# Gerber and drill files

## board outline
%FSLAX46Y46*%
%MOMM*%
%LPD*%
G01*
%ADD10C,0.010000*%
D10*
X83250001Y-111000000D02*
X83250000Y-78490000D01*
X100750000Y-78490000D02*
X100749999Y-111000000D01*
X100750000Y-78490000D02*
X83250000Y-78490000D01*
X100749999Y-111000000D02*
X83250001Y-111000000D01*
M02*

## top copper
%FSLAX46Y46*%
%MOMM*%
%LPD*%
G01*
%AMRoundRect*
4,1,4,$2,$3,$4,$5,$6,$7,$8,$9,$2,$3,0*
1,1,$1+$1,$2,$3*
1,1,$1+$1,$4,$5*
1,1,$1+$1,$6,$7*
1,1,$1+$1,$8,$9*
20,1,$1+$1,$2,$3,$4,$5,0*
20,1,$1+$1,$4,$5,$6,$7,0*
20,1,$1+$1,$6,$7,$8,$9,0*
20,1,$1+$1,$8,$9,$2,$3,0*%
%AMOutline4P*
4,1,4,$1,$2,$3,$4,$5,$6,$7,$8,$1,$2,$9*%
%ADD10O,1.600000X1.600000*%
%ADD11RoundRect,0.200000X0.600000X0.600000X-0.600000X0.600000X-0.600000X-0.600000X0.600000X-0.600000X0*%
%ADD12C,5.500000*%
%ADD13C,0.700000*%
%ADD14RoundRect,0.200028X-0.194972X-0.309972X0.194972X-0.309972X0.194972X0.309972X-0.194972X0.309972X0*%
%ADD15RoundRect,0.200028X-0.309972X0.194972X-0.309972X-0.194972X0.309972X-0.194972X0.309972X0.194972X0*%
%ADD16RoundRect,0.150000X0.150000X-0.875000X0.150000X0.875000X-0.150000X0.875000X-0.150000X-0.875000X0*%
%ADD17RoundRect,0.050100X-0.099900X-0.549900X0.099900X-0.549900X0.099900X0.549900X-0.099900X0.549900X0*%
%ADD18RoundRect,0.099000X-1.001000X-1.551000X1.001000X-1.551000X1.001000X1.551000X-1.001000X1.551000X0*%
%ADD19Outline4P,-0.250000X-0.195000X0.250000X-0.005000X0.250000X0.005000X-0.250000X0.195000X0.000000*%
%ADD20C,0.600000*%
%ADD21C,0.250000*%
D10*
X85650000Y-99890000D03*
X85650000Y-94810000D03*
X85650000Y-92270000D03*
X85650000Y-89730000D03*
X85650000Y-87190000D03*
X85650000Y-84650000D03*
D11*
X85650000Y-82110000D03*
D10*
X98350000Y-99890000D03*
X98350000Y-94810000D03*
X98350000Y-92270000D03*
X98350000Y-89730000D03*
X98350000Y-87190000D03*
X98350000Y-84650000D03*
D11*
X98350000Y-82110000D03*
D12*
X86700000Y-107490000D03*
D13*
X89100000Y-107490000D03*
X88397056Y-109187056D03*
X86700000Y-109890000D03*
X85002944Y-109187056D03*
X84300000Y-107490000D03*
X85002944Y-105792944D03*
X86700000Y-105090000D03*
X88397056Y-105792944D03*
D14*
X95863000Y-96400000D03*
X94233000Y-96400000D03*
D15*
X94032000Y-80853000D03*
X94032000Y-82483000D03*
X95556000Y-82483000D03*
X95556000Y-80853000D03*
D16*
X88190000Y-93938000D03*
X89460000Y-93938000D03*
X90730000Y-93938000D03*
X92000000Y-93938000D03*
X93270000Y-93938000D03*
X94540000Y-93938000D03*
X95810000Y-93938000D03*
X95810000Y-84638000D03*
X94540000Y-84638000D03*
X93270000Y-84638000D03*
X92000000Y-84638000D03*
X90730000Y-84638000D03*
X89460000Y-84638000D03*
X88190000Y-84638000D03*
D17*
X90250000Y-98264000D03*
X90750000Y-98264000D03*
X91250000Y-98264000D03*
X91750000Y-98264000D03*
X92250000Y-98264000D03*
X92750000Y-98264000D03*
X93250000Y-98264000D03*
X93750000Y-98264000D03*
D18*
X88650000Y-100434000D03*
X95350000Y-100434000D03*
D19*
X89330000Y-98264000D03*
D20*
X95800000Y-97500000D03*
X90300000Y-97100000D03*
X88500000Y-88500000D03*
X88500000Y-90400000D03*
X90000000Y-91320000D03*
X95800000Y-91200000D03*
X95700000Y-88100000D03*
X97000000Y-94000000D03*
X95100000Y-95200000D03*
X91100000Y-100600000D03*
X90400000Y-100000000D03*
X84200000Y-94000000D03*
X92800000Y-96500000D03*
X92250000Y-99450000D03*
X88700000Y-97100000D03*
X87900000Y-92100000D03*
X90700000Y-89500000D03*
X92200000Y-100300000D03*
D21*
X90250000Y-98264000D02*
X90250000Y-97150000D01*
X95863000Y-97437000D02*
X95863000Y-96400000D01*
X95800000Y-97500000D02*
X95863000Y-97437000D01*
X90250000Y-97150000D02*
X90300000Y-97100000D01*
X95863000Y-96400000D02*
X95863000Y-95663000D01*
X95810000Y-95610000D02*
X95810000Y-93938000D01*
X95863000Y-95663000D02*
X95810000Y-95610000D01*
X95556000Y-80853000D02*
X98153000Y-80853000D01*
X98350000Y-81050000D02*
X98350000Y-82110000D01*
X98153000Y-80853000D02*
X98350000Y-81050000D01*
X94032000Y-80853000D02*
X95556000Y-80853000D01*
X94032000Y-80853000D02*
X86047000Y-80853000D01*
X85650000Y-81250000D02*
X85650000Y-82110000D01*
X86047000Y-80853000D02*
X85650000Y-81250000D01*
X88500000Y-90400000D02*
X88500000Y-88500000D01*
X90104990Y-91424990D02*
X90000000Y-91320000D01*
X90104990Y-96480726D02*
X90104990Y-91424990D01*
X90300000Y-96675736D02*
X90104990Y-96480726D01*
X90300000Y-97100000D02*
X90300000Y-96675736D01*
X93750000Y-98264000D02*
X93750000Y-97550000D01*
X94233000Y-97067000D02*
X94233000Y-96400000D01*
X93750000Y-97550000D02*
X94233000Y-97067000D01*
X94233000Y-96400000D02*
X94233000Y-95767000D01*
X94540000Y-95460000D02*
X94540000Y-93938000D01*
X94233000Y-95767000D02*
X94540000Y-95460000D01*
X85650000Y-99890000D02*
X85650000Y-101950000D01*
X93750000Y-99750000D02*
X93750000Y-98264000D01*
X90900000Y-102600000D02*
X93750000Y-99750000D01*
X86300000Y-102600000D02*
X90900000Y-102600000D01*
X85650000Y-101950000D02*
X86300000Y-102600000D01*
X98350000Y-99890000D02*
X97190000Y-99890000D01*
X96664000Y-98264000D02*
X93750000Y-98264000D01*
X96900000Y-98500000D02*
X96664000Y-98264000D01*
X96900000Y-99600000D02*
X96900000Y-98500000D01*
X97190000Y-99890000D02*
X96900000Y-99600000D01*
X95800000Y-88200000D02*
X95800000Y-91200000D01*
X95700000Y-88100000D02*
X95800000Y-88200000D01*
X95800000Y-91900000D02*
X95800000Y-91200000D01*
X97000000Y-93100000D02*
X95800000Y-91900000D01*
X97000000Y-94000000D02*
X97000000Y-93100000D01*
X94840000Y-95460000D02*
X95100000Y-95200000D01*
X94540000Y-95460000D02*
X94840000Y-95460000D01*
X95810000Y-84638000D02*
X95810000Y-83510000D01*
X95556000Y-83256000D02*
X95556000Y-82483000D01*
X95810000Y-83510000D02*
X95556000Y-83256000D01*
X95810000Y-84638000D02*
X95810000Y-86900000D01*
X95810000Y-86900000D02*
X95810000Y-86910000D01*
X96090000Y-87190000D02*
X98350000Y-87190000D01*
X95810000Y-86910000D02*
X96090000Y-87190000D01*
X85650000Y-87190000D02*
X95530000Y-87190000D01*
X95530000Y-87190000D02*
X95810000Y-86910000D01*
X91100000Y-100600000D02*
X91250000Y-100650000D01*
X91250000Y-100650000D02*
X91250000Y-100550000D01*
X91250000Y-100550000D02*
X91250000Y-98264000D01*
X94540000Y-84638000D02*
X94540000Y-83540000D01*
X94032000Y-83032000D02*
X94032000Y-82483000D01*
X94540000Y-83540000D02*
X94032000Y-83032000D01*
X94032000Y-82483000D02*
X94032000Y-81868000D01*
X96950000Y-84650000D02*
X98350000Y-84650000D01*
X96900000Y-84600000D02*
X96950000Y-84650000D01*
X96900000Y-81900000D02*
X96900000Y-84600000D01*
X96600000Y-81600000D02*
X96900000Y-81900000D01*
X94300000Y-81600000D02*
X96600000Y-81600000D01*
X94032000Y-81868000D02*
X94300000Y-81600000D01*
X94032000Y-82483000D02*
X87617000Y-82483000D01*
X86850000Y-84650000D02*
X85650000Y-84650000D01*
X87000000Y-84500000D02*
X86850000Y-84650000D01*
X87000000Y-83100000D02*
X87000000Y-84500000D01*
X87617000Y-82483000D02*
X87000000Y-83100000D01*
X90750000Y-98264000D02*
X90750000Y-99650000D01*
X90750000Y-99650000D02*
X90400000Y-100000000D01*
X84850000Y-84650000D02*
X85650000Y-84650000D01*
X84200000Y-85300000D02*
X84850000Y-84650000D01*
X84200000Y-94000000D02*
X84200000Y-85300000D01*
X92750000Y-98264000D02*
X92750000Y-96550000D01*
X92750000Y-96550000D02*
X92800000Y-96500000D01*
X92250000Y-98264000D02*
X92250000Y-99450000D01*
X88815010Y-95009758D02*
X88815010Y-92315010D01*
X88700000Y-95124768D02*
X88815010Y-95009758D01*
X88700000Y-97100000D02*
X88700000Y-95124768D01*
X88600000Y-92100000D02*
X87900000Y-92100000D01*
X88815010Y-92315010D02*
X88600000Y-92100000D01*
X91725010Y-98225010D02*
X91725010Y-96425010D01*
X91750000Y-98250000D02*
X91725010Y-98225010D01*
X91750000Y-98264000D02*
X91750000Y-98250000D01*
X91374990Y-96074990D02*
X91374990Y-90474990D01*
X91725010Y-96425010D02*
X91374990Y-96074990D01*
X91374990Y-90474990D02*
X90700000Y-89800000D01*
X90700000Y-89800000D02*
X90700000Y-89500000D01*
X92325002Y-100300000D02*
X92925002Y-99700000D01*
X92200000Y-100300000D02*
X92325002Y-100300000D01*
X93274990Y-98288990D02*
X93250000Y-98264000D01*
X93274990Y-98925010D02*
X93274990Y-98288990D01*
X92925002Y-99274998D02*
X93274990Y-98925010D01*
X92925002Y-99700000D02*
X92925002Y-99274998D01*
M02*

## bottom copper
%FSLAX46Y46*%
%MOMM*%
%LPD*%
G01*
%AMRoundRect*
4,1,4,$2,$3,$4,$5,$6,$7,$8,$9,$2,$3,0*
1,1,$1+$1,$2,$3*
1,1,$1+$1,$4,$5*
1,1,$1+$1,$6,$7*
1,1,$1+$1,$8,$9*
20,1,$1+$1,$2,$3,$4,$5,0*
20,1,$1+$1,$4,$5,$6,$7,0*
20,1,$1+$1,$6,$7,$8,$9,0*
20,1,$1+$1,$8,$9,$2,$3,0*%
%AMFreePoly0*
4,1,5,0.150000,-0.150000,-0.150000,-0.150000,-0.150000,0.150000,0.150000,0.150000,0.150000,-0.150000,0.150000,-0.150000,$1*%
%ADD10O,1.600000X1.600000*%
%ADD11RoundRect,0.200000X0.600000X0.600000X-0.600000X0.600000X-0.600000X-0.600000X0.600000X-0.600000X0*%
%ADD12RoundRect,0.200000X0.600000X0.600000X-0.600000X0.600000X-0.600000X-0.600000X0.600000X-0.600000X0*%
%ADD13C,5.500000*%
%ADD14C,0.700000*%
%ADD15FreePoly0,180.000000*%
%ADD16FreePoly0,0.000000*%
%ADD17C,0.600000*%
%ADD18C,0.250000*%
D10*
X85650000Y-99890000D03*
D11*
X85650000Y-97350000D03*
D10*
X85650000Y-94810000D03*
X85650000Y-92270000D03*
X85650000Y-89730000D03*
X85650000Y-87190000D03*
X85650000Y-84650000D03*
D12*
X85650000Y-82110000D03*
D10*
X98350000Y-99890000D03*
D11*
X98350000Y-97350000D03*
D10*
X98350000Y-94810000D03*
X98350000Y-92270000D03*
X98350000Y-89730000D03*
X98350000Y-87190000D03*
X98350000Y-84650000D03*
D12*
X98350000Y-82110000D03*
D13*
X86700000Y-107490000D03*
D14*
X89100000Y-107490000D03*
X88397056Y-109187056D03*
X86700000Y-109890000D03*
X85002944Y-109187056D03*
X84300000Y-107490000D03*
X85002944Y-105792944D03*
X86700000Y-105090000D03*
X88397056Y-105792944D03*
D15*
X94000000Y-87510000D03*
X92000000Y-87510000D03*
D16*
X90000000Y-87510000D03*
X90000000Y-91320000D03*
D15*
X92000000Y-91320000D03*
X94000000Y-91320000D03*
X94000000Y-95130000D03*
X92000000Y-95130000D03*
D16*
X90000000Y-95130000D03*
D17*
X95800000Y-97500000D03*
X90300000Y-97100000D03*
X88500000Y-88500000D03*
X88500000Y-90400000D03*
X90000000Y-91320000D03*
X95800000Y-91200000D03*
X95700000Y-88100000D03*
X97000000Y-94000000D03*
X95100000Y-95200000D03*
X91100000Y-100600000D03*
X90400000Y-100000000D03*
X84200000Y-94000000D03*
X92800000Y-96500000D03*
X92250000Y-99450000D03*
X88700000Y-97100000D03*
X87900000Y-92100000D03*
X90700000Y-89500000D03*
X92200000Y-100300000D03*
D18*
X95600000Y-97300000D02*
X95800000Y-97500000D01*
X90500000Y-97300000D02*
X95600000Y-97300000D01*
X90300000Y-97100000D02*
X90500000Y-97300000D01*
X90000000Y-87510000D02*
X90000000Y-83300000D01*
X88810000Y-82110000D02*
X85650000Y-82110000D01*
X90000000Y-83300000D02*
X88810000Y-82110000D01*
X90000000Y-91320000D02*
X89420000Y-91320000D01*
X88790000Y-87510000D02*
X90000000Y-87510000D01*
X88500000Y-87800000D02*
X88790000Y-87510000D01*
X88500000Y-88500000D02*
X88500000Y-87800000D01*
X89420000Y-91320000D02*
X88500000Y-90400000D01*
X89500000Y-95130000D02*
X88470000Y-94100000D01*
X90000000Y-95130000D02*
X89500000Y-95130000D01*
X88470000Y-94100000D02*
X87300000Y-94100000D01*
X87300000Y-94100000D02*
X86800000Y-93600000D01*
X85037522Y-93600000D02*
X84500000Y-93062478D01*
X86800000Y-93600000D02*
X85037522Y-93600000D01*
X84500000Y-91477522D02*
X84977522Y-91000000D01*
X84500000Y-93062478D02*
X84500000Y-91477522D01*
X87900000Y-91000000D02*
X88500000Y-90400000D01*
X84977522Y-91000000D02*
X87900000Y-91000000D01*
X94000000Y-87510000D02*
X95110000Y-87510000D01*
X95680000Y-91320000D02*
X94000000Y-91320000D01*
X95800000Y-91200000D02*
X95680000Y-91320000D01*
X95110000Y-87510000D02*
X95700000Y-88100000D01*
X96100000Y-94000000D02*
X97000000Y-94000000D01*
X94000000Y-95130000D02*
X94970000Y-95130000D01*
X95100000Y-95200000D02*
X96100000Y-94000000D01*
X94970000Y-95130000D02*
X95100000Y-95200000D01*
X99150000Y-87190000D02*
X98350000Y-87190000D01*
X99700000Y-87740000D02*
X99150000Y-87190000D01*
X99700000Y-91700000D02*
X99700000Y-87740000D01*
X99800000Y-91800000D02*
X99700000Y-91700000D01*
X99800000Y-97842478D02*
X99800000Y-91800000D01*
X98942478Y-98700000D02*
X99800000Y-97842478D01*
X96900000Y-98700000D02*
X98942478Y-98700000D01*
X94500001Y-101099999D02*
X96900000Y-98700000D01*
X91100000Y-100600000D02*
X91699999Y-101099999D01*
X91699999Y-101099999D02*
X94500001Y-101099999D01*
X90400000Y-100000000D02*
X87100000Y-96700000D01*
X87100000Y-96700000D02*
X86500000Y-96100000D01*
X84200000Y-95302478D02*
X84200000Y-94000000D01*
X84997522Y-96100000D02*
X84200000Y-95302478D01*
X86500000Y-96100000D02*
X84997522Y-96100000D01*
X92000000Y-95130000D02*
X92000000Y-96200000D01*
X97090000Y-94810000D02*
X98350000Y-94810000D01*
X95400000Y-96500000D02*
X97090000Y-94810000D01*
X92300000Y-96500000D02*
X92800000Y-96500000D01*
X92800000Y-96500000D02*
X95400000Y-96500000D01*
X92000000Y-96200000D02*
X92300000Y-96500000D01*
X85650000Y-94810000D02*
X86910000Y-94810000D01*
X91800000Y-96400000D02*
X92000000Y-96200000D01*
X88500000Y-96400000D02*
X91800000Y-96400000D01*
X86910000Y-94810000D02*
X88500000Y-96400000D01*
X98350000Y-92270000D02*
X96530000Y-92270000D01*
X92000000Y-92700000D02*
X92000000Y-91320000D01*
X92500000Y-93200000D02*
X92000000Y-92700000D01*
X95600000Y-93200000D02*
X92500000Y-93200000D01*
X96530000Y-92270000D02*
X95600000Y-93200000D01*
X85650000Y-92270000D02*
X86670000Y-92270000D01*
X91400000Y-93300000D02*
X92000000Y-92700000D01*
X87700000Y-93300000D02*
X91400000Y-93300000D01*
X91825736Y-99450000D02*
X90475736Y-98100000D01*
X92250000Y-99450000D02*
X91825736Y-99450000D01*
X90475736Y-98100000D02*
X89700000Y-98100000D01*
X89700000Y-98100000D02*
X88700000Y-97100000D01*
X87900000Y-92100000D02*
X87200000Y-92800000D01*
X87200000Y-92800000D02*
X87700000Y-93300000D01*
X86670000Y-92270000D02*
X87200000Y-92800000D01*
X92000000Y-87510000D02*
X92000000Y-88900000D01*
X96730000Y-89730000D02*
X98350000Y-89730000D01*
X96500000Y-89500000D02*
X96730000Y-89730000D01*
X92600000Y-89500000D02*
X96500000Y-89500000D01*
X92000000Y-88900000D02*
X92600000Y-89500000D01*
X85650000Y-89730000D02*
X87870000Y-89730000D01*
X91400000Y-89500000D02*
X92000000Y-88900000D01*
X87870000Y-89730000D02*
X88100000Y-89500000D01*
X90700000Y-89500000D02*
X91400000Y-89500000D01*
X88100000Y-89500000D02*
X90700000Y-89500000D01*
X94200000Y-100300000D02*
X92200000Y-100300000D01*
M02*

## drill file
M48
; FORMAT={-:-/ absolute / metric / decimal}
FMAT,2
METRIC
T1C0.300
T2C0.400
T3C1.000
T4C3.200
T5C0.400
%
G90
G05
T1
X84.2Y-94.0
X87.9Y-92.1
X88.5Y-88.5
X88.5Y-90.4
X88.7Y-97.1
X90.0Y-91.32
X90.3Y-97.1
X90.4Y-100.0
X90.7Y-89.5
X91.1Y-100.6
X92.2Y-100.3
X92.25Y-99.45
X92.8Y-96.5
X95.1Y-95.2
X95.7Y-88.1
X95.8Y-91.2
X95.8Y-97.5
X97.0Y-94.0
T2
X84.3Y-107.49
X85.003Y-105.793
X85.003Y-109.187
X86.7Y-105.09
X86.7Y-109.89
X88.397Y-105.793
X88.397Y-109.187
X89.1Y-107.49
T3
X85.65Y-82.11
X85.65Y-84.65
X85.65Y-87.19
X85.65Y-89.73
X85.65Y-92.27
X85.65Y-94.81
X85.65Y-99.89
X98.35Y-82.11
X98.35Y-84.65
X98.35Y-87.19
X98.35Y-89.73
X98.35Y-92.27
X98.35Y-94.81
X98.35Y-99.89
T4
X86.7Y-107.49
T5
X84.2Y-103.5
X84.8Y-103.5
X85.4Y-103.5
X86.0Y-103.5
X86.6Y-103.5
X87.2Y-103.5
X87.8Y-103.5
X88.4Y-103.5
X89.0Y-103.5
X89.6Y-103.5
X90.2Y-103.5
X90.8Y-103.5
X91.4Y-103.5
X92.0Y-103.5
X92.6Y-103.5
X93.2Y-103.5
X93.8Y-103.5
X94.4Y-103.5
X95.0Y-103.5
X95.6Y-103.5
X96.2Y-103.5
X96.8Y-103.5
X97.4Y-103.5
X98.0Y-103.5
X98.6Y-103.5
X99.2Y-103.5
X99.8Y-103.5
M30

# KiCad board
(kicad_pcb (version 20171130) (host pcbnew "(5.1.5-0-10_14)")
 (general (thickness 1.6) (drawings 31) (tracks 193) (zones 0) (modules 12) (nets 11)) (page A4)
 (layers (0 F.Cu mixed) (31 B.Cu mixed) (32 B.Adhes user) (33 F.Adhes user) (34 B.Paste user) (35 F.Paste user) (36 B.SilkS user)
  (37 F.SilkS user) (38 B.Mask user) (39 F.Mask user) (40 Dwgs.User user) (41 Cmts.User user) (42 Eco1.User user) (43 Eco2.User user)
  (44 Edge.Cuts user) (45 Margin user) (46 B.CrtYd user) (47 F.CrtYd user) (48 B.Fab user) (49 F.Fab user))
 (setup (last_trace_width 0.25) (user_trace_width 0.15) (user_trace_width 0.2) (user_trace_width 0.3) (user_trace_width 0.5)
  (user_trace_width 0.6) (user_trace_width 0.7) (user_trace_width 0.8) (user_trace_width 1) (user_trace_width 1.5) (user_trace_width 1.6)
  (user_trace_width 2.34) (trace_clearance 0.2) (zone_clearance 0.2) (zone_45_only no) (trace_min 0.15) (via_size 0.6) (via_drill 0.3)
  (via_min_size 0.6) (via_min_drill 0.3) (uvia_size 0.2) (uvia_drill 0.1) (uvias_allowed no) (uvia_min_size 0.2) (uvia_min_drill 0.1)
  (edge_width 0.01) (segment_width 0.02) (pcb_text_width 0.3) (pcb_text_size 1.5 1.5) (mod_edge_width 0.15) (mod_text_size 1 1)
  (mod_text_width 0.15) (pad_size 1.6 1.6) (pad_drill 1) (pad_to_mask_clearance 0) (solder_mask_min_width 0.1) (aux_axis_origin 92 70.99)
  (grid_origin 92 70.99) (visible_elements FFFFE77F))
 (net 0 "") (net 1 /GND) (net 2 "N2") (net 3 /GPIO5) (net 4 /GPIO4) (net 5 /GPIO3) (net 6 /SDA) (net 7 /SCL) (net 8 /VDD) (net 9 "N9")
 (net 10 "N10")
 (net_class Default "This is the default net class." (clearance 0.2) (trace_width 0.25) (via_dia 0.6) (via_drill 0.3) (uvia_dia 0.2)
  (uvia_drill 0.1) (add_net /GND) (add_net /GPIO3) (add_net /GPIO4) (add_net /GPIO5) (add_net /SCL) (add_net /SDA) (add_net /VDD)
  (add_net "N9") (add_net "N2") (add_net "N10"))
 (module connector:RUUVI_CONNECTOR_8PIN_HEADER (layer B.Cu) (at 85.65 82.11 180)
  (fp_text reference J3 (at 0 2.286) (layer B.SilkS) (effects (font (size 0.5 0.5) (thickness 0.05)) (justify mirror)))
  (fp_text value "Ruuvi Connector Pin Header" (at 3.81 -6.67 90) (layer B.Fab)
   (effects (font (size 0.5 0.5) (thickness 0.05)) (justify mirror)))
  (pad 8 thru_hole oval (at 0 -17.78 180) (size 1.6 1.6) (drill 1) (layers *.Cu *.Mask) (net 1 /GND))
  (pad 7 smd roundrect (at 0 -15.24 180) (size 1.6 1.6) (layers B.Cu B.Paste B.Mask) (roundrect_rratio 0.125) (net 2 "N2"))
  (pad 6 thru_hole oval (at 0 -12.7 180) (size 1.6 1.6) (drill 1) (layers *.Cu *.Mask) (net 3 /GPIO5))
  (pad 5 thru_hole oval (at 0 -10.16 180) (size 1.6 1.6) (drill 1) (layers *.Cu *.Mask) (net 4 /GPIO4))
  (pad 4 thru_hole oval (at 0 -7.62 180) (size 1.6 1.6) (drill 1) (layers *.Cu *.Mask) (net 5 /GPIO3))
  (pad 3 thru_hole oval (at 0 -5.08 180) (size 1.6 1.6) (drill 1) (layers *.Cu *.Mask) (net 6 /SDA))
  (pad 2 thru_hole oval (at 0 -2.54 180) (size 1.6 1.6) (drill 1) (layers *.Cu *.Mask) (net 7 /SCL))
  (pad 1 thru_hole roundrect (at 0 0 180) (size 1.6 1.6) (drill 1) (layers *.Cu *.Mask) (roundrect_rratio 0.125) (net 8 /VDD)))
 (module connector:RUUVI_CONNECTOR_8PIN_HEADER (layer B.Cu) (at 98.35 82.11 180)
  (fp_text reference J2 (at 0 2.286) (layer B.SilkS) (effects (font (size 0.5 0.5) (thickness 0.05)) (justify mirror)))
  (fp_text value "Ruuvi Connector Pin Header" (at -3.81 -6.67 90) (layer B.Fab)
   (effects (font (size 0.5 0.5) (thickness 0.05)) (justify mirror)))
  (pad 8 thru_hole oval (at 0 -17.78 180) (size 1.6 1.6) (drill 1) (layers *.Cu *.Mask) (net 1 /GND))
  (pad 7 smd roundrect (at 0 -15.24 180) (size 1.6 1.6) (layers B.Cu B.Paste B.Mask) (roundrect_rratio 0.125) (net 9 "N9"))
  (pad 6 thru_hole oval (at 0 -12.7 180) (size 1.6 1.6) (drill 1) (layers *.Cu *.Mask) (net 3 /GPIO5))
  (pad 5 thru_hole oval (at 0 -10.16 180) (size 1.6 1.6) (drill 1) (layers *.Cu *.Mask) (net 4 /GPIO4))
  (pad 4 thru_hole oval (at 0 -7.62 180) (size 1.6 1.6) (drill 1) (layers *.Cu *.Mask) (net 5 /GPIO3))
  (pad 3 thru_hole oval (at 0 -5.08 180) (size 1.6 1.6) (drill 1) (layers *.Cu *.Mask) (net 6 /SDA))
  (pad 2 thru_hole oval (at 0 -2.54 180) (size 1.6 1.6) (drill 1) (layers *.Cu *.Mask) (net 7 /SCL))
  (pad 1 thru_hole roundrect (at 0 0 180) (size 1.6 1.6) (drill 1) (layers *.Cu *.Mask) (roundrect_rratio 0.125) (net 8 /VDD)))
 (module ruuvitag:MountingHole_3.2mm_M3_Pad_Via (layer F.Cu) (at 86.7 107.49)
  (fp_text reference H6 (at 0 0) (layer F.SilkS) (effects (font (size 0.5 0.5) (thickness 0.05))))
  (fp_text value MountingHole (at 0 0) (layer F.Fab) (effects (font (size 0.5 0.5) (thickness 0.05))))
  (pad 1 thru_hole circle (at 0 0) (size 5.5 5.5) (drill 3.2) (layers *.Cu *.Mask))
  (pad 1 thru_hole circle (at 2.4 0) (size 0.7 0.7) (drill 0.4) (layers *.Cu *.Mask))
  (pad 1 thru_hole circle (at 1.697056 1.697056) (size 0.7 0.7) (drill 0.4) (layers *.Cu *.Mask))
  (pad 1 thru_hole circle (at 0 2.4) (size 0.7 0.7) (drill 0.4) (layers *.Cu *.Mask))
  (pad 1 thru_hole circle (at -1.697056 1.697056) (size 0.7 0.7) (drill 0.4) (layers *.Cu *.Mask))
  (pad 1 thru_hole circle (at -2.4 0) (size 0.7 0.7) (drill 0.4) (layers *.Cu *.Mask))
  (pad 1 thru_hole circle (at -1.697056 -1.697056) (size 0.7 0.7) (drill 0.4) (layers *.Cu *.Mask))
  (pad 1 thru_hole circle (at 0 -2.4) (size 0.7 0.7) (drill 0.4) (layers *.Cu *.Mask))
  (pad 1 thru_hole circle (at 1.697056 -1.697056) (size 0.7 0.7) (drill 0.4) (layers *.Cu *.Mask)))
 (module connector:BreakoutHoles (layer F.Cu) (at 92 103.5)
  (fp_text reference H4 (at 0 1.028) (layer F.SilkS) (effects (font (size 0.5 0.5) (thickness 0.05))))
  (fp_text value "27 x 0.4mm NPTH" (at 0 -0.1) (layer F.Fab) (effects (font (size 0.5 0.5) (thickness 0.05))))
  (pad "" np_thru_hole circle (at -6.6 0) (size 0.4 0.4) (drill 0.4) (layers *.Cu *.Mask))
  (pad "" np_thru_hole circle (at -0.6 0) (size 0.4 0.4) (drill 0.4) (layers *.Cu *.Mask))
  (pad "" np_thru_hole circle (at -3.6 0) (size 0.4 0.4) (drill 0.4) (layers *.Cu *.Mask))
  (pad "" np_thru_hole circle (at -1.2 0) (size 0.4 0.4) (drill 0.4) (layers *.Cu *.Mask))
  (pad "" np_thru_hole circle (at -3 0) (size 0.4 0.4) (drill 0.4) (layers *.Cu *.Mask))
  (pad "" np_thru_hole circle (at -1.8 0) (size 0.4 0.4) (drill 0.4) (layers *.Cu *.Mask))
  (pad "" np_thru_hole circle (at -4.8 0) (size 0.4 0.4) (drill 0.4) (layers *.Cu *.Mask))
  (pad "" np_thru_hole circle (at -5.4 0) (size 0.4 0.4) (drill 0.4) (layers *.Cu *.Mask))
  (pad "" np_thru_hole circle (at -7.8 0) (size 0.4 0.4) (drill 0.4) (layers *.Cu *.Mask))
  (pad "" np_thru_hole circle (at -2.4 0) (size 0.4 0.4) (drill 0.4) (layers *.Cu *.Mask))
  (pad "" np_thru_hole circle (at -4.2 0) (size 0.4 0.4) (drill 0.4) (layers *.Cu *.Mask))
  (pad "" np_thru_hole circle (at -7.2 0) (size 0.4 0.4) (drill 0.4) (layers *.Cu *.Mask))
  (pad "" np_thru_hole circle (at -6 0) (size 0.4 0.4) (drill 0.4) (layers *.Cu *.Mask))
  (pad "" np_thru_hole circle (at 7.8 0) (size 0.4 0.4) (drill 0.4) (layers *.Cu *.Mask))
  (pad "" np_thru_hole circle (at 7.2 0) (size 0.4 0.4) (drill 0.4) (layers *.Cu *.Mask))
  (pad "" np_thru_hole circle (at 6.6 0) (size 0.4 0.4) (drill 0.4) (layers *.Cu *.Mask))
  (pad "" np_thru_hole circle (at 6 0) (size 0.4 0.4) (drill 0.4) (layers *.Cu *.Mask))
  (pad "" np_thru_hole circle (at 5.4 0) (size 0.4 0.4) (drill 0.4) (layers *.Cu *.Mask))
  (pad "" np_thru_hole circle (at 4.8 0) (size 0.4 0.4) (drill 0.4) (layers *.Cu *.Mask))
  (pad "" np_thru_hole circle (at 4.2 0) (size 0.4 0.4) (drill 0.4) (layers *.Cu *.Mask))
  (pad "" np_thru_hole circle (at 3.6 0) (size 0.4 0.4) (drill 0.4) (layers *.Cu *.Mask))
  (pad "" np_thru_hole circle (at 3 0) (size 0.4 0.4) (drill 0.4) (layers *.Cu *.Mask))
  (pad "" np_thru_hole circle (at 2.4 0) (size 0.4 0.4) (drill 0.4) (layers *.Cu *.Mask))
  (pad "" np_thru_hole circle (at 1.8 0) (size 0.4 0.4) (drill 0.4) (layers *.Cu *.Mask))
  (pad "" np_thru_hole circle (at 1.2 0) (size 0.4 0.4) (drill 0.4) (layers *.Cu *.Mask))
  (pad "" np_thru_hole circle (at 0.6 0) (size 0.4 0.4) (drill 0.4) (layers *.Cu *.Mask))
  (pad "" np_thru_hole circle (at 0 0) (size 0.4 0.4) (drill 0.4) (layers *.Cu *.Mask)))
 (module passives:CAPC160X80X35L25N (layer F.Cu) (at 95.048 96.4)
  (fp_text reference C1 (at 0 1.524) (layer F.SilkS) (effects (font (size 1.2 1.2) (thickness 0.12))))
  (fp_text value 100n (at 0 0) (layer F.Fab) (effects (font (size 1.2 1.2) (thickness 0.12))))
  (pad 2 smd roundrect (at 0.815 0) (size 0.79 1.02) (layers F.Cu F.Paste F.Mask) (roundrect_rratio 0.2532) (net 8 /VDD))
  (pad 1 smd roundrect (at -0.815 0) (size 0.79 1.02) (layers F.Cu F.Paste F.Mask) (roundrect_rratio 0.2532) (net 1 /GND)))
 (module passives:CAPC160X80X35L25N (layer F.Cu) (at 94.032 81.668 270)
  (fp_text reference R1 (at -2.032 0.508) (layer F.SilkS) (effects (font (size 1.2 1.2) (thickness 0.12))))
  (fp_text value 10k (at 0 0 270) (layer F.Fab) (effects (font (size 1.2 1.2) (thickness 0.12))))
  (pad 1 smd roundrect (at -0.815 0 270) (size 0.79 1.02) (layers F.Cu F.Paste F.Mask) (roundrect_rratio 0.2532) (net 8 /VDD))
  (pad 2 smd roundrect (at 0.815 0 270) (size 0.79 1.02) (layers F.Cu F.Paste F.Mask) (roundrect_rratio 0.2532) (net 7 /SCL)))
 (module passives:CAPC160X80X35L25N (layer F.Cu) (at 95.556 81.668 270)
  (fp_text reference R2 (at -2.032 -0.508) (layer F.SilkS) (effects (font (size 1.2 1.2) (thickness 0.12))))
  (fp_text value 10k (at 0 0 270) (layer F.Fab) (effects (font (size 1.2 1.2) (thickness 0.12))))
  (pad 2 smd roundrect (at 0.815 0 270) (size 0.79 1.02) (layers F.Cu F.Paste F.Mask) (roundrect_rratio 0.2532) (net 6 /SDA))
  (pad 1 smd roundrect (at -0.815 0 270) (size 0.79 1.02) (layers F.Cu F.Paste F.Mask) (roundrect_rratio 0.2532) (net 8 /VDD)))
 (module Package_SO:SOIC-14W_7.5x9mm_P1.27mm (layer F.Cu) (at 92 89.288 90)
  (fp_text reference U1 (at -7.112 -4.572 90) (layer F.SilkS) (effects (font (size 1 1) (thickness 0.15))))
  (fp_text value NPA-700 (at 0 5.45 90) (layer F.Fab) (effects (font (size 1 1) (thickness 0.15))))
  (pad 1 smd roundrect (at -4.65 -3.81 90) (size 2.05 0.6) (layers F.Cu F.Paste F.Mask) (roundrect_rratio 0.25))
  (pad 2 smd roundrect (at -4.65 -2.54 90) (size 2.05 0.6) (layers F.Cu F.Paste F.Mask) (roundrect_rratio 0.25))
  (pad 3 smd roundrect (at -4.65 -1.27 90) (size 2.05 0.6) (layers F.Cu F.Paste F.Mask) (roundrect_rratio 0.25))
  (pad 4 smd roundrect (at -4.65 0 90) (size 2.05 0.6) (layers F.Cu F.Paste F.Mask) (roundrect_rratio 0.25))
  (pad 5 smd roundrect (at -4.65 1.27 90) (size 2.05 0.6) (layers F.Cu F.Paste F.Mask) (roundrect_rratio 0.25))
  (pad 6 smd roundrect (at -4.65 2.54 90) (size 2.05 0.6) (layers F.Cu F.Paste F.Mask) (roundrect_rratio 0.25) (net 1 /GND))
  (pad 7 smd roundrect (at -4.65 3.81 90) (size 2.05 0.6) (layers F.Cu F.Paste F.Mask) (roundrect_rratio 0.25) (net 8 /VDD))
  (pad 8 smd roundrect (at 4.65 3.81 90) (size 2.05 0.6) (layers F.Cu F.Paste F.Mask) (roundrect_rratio 0.25) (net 6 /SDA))
  (pad 9 smd roundrect (at 4.65 2.54 90) (size 2.05 0.6) (layers F.Cu F.Paste F.Mask) (roundrect_rratio 0.25) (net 7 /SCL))
  (pad 10 smd roundrect (at 4.65 1.27 90) (size 2.05 0.6) (layers F.Cu F.Paste F.Mask) (roundrect_rratio 0.25))
  (pad 11 smd roundrect (at 4.65 0 90) (size 2.05 0.6) (layers F.Cu F.Paste F.Mask) (roundrect_rratio 0.25))
  (pad 12 smd roundrect (at 4.65 -1.27 90) (size 2.05 0.6) (layers F.Cu F.Paste F.Mask) (roundrect_rratio 0.25))
  (pad 13 smd roundrect (at 4.65 -2.54 90) (size 2.05 0.6) (layers F.Cu F.Paste F.Mask) (roundrect_rratio 0.25))
  (pad 14 smd roundrect (at 4.65 -3.81 90) (size 2.05 0.6) (layers F.Cu F.Paste F.Mask) (roundrect_rratio 0.25)))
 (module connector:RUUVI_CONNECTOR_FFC (layer F.Cu) (at 92 100.464)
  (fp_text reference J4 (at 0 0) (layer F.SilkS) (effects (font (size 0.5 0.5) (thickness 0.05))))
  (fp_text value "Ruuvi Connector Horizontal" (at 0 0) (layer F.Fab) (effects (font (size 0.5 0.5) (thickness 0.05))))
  (pad 1 smd roundrect (at -1.75 -2.2) (size 0.3 1.2) (layers F.Cu F.Paste F.Mask) (roundrect_rratio 0.167) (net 8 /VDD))
  (pad 2 smd roundrect (at -1.25 -2.2) (size 0.3 1.2) (layers F.Cu F.Paste F.Mask) (roundrect_rratio 0.167) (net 7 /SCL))
  (pad 3 smd roundrect (at -0.75 -2.2) (size 0.3 1.2) (layers F.Cu F.Paste F.Mask) (roundrect_rratio 0.167) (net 6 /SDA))
  (pad 4 smd roundrect (at -0.25 -2.2) (size 0.3 1.2) (layers F.Cu F.Paste F.Mask) (roundrect_rratio 0.167) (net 5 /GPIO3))
  (pad 5 smd roundrect (at 0.25 -2.2) (size 0.3 1.2) (layers F.Cu F.Paste F.Mask) (roundrect_rratio 0.167) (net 4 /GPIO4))
  (pad 6 smd roundrect (at 0.75 -2.2) (size 0.3 1.2) (layers F.Cu F.Paste F.Mask) (roundrect_rratio 0.167) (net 3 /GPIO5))
  (pad 7 smd roundrect (at 1.25 -2.2) (size 0.3 1.2) (layers F.Cu F.Paste F.Mask) (roundrect_rratio 0.167) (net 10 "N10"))
  (pad 8 smd roundrect (at 1.75 -2.2) (size 0.3 1.2) (layers F.Cu F.Paste F.Mask) (roundrect_rratio 0.167) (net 1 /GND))
  (pad ~ smd roundrect (at -3.35 -0.03) (size 2.2 3.3) (layers F.Cu F.Paste F.Mask) (roundrect_rratio 0.045))
  (pad ~ smd roundrect (at 3.35 -0.03) (size 2.2 3.3) (layers F.Cu F.Paste F.Mask) (roundrect_rratio 0.045))
  (pad ~ smd trapezoid (at -2.67 -2.2) (size 0.5 0.2) (rect_delta 0.19 0) (layers F.Cu F.Mask)))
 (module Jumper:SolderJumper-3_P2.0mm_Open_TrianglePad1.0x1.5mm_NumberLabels (layer B.Cu) (at 92 87.51 180)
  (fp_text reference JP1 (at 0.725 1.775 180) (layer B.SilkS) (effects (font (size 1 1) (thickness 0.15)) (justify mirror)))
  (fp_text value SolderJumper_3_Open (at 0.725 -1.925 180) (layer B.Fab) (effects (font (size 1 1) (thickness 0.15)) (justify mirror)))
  (pad "" smd rect (at 1.2 0 180) (size 1.5 1.5) (layers B.Mask))
  (pad "" smd rect (at -1.2 0 180) (size 1.5 1.5) (layers B.Mask))
  (pad 1 smd custom (at -2 0 180) (size 0.3 0.3) (layers B.Cu B.Mask) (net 1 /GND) (zone_connect 2)
   (options (clearance outline) (anchor rect)) (primitives))
  (pad 2 smd custom (at 0 0 180) (size 0.3 0.3) (layers B.Cu) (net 5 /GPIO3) (zone_connect 2) (options (clearance outline) (anchor rect))
   (primitives))
  (pad 3 smd custom (at 2 0) (size 0.3 0.3) (layers B.Cu B.Mask) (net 8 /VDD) (zone_connect 2) (options (clearance outline) (anchor rect))
   (primitives)))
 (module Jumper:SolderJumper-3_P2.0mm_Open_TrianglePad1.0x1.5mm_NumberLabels (layer B.Cu) (at 92 91.32 180)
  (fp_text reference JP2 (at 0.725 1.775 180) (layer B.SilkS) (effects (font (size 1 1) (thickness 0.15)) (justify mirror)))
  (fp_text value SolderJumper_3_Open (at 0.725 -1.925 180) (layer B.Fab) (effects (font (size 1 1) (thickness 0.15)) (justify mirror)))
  (pad 3 smd custom (at 2 0) (size 0.3 0.3) (layers B.Cu B.Mask) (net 8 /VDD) (zone_connect 2) (options (clearance outline) (anchor rect))
   (primitives))
  (pad 2 smd custom (at 0 0 180) (size 0.3 0.3) (layers B.Cu) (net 4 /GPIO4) (zone_connect 2) (options (clearance outline) (anchor rect))
   (primitives))
  (pad 1 smd custom (at -2 0 180) (size 0.3 0.3) (layers B.Cu B.Mask) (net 1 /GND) (zone_connect 2)
   (options (clearance outline) (anchor rect)) (primitives))
  (pad "" smd rect (at -1.2 0 180) (size 1.5 1.5) (layers B.Mask))
  (pad "" smd rect (at 1.2 0 180) (size 1.5 1.5) (layers B.Mask)))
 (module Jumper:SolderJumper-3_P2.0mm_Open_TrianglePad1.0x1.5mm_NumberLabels (layer B.Cu) (at 92 95.13 180)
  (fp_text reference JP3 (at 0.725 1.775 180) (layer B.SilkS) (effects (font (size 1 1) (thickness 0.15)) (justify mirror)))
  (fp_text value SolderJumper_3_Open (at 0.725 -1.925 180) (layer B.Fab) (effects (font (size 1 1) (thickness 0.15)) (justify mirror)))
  (pad "" smd rect (at 1.2 0 180) (size 1.5 1.5) (layers B.Mask))
  (pad "" smd rect (at -1.2 0 180) (size 1.5 1.5) (layers B.Mask))
  (pad 1 smd custom (at -2 0 180) (size 0.3 0.3) (layers B.Cu B.Mask) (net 1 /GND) (zone_connect 2)
   (options (clearance outline) (anchor rect)) (primitives))
  (pad 2 smd custom (at 0 0 180) (size 0.3 0.3) (layers B.Cu) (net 3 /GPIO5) (zone_connect 2) (options (clearance outline) (anchor rect))
   (primitives))
  (pad 3 smd custom (at 2 0) (size 0.3 0.3) (layers B.Cu B.Mask) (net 8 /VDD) (zone_connect 2) (options (clearance outline) (anchor rect))
   (primitives)))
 (gr_line (start 83.250001 111) (end 83.25 78.49) (layer Edge.Cuts) (width 0.01))
 (gr_line (start 100.75 78.49) (end 100.749999 111) (layer Edge.Cuts) (width 0.01))
 (gr_line (start 100.75 78.49) (end 83.25 78.49) (layer Edge.Cuts) (width 0.01))
 (gr_line (start 100.749999 111) (end 83.250001 111) (layer Edge.Cuts) (width 0.01))
 (segment (start 90.25 98.264) (end 90.25 97.15) (width 0.25) (layer F.Cu) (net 8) (status 400000))
 (segment (start 95.863 97.437) (end 95.863 96.4) (width 0.25) (layer F.Cu) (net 8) (status 800000))
 (segment (start 95.8 97.5) (end 95.863 97.437) (width 0.25) (layer F.Cu) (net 8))
 (via (at 95.8 97.5) (size 0.6) (drill 0.3) (layers F.Cu B.Cu) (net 8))
 (segment (start 95.6 97.3) (end 95.8 97.5) (width 0.25) (layer B.Cu) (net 8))
 (segment (start 90.5 97.3) (end 95.6 97.3) (width 0.25) (layer B.Cu) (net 8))
 (segment (start 90.3 97.1) (end 90.5 97.3) (width 0.25) (layer B.Cu) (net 8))
 (via (at 90.3 97.1) (size 0.6) (drill 0.3) (layers F.Cu B.Cu) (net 8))
 (segment (start 90.25 97.15) (end 90.3 97.1) (width 0.25) (layer F.Cu) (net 8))
 (segment (start 95.863 96.4) (end 95.863 95.663) (width 0.25) (layer F.Cu) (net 8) (status 400000))
 (segment (start 95.81 95.61) (end 95.81 93.938) (width 0.25) (layer F.Cu) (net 8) (status 800000))
 (segment (start 95.863 95.663) (end 95.81 95.61) (width 0.25) (layer F.Cu) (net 8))
 (segment (start 95.556 80.853) (end 98.153 80.853) (width 0.25) (layer F.Cu) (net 8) (status 400000))
 (segment (start 98.35 81.05) (end 98.35 82.11) (width 0.25) (layer F.Cu) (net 8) (status 800000))
 (segment (start 98.153 80.853) (end 98.35 81.05) (width 0.25) (layer F.Cu) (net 8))
 (segment (start 94.032 80.853) (end 95.556 80.853) (width 0.25) (layer F.Cu) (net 8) (status C00000))
 (segment (start 94.032 80.853) (end 86.047 80.853) (width 0.25) (layer F.Cu) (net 8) (status 400000))
 (segment (start 85.65 81.25) (end 85.65 82.11) (width 0.25) (layer F.Cu) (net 8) (status 800000))
 (segment (start 86.047 80.853) (end 85.65 81.25) (width 0.25) (layer F.Cu) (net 8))
 (segment (start 90 87.51) (end 90 83.3) (width 0.25) (layer B.Cu) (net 8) (status 400000))
 (segment (start 88.81 82.11) (end 85.65 82.11) (width 0.25) (layer B.Cu) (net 8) (status 800000))
 (segment (start 90 83.3) (end 88.81 82.11) (width 0.25) (layer B.Cu) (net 8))
 (segment (start 90 91.32) (end 89.42 91.32) (width 0.25) (layer B.Cu) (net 8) (status 400000))
 (segment (start 88.79 87.51) (end 90 87.51) (width 0.25) (layer B.Cu) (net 8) (status 800000))
 (segment (start 88.5 87.8) (end 88.79 87.51) (width 0.25) (layer B.Cu) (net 8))
 (segment (start 88.5 88.5) (end 88.5 87.8) (width 0.25) (layer B.Cu) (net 8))
 (via (at 88.5 88.5) (size 0.6) (drill 0.3) (layers F.Cu B.Cu) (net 8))
 (segment (start 88.5 90.4) (end 88.5 88.5) (width 0.25) (layer F.Cu) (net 8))
 (via (at 88.5 90.4) (size 0.6) (drill 0.3) (layers F.Cu B.Cu) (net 8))
 (segment (start 89.42 91.32) (end 88.5 90.4) (width 0.25) (layer B.Cu) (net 8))
 (via (at 90 91.32) (size 0.6) (drill 0.3) (layers F.Cu B.Cu) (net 8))
 (segment (start 90.10499 91.42499) (end 90 91.32) (width 0.25) (layer F.Cu) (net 8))
 (segment (start 90.10499 96.480726) (end 90.10499 91.42499) (width 0.25) (layer F.Cu) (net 8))
 (segment (start 90.3 96.675736) (end 90.10499 96.480726) (width 0.25) (layer F.Cu) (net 8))
 (segment (start 90.3 97.1) (end 90.3 96.675736) (width 0.25) (layer F.Cu) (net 8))
 (segment (start 89.5 95.13) (end 88.47 94.1) (width 0.25) (layer B.Cu) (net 8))
 (segment (start 90 95.13) (end 89.5 95.13) (width 0.25) (layer B.Cu) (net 8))
 (segment (start 88.47 94.1) (end 87.3 94.1) (width 0.25) (layer B.Cu) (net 8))
 (segment (start 87.3 94.1) (end 86.8 93.6) (width 0.25) (layer B.Cu) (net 8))
 (segment (start 85.037522 93.6) (end 84.5 93.062478) (width 0.25) (layer B.Cu) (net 8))
 (segment (start 86.8 93.6) (end 85.037522 93.6) (width 0.25) (layer B.Cu) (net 8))
 (segment (start 84.5 91.477522) (end 84.977522 91) (width 0.25) (layer B.Cu) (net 8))
 (segment (start 84.5 93.062478) (end 84.5 91.477522) (width 0.25) (layer B.Cu) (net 8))
 (segment (start 87.9 91) (end 88.5 90.4) (width 0.25) (layer B.Cu) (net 8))
 (segment (start 84.977522 91) (end 87.9 91) (width 0.25) (layer B.Cu) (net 8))
 (segment (start 93.75 98.264) (end 93.75 97.55) (width 0.25) (layer F.Cu) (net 1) (status 400000))
 (segment (start 94.233 97.067) (end 94.233 96.4) (width 0.25) (layer F.Cu) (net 1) (status 800000))
 (segment (start 93.75 97.55) (end 94.233 97.067) (width 0.25) (layer F.Cu) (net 1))
 (segment (start 94.233 96.4) (end 94.233 95.767) (width 0.25) (layer F.Cu) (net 1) (status 400000))
 (segment (start 94.54 95.46) (end 94.54 93.938) (width 0.25) (layer F.Cu) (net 1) (status 800000))
 (segment (start 94.233 95.767) (end 94.54 95.46) (width 0.25) (layer F.Cu) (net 1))
 (segment (start 85.65 99.89) (end 85.65 101.95) (width 0.25) (layer F.Cu) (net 1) (status 400000))
 (segment (start 93.75 99.75) (end 93.75 98.264) (width 0.25) (layer F.Cu) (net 1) (status 800000))
 (segment (start 90.9 102.6) (end 93.75 99.75) (width 0.25) (layer F.Cu) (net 1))
 (segment (start 86.3 102.6) (end 90.9 102.6) (width 0.25) (layer F.Cu) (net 1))
 (segment (start 85.65 101.95) (end 86.3 102.6) (width 0.25) (layer F.Cu) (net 1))
 (segment (start 98.35 99.89) (end 97.19 99.89) (width 0.25) (layer F.Cu) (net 1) (status 400000))
 (segment (start 96.664 98.264) (end 93.75 98.264) (width 0.25) (layer F.Cu) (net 1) (status 800000))
 (segment (start 96.9 98.5) (end 96.664 98.264) (width 0.25) (layer F.Cu) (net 1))
 (segment (start 96.9 99.6) (end 96.9 98.5) (width 0.25) (layer F.Cu) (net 1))
 (segment (start 97.19 99.89) (end 96.9 99.6) (width 0.25) (layer F.Cu) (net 1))
 (segment (start 94 87.51) (end 95.11 87.51) (width 0.25) (layer B.Cu) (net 1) (status 400000))
 (segment (start 95.68 91.32) (end 94 91.32) (width 0.25) (layer B.Cu) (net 1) (status 800000))
 (segment (start 95.8 91.2) (end 95.68 91.32) (width 0.25) (layer B.Cu) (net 1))
 (via (at 95.8 91.2) (size 0.6) (drill 0.3) (layers F.Cu B.Cu) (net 1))
 (segment (start 95.8 88.2) (end 95.8 91.2) (width 0.25) (layer F.Cu) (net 1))
 (segment (start 95.7 88.1) (end 95.8 88.2) (width 0.25) (layer F.Cu) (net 1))
 (via (at 95.7 88.1) (size 0.6) (drill 0.3) (layers F.Cu B.Cu) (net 1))
 (segment (start 95.11 87.51) (end 95.7 88.1) (width 0.25) (layer B.Cu) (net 1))
 (segment (start 95.8 91.9) (end 95.8 91.2) (width 0.25) (layer F.Cu) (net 1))
 (segment (start 97 93.1) (end 95.8 91.9) (width 0.25) (layer F.Cu) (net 1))
 (segment (start 97 94) (end 97 93.1) (width 0.25) (layer F.Cu) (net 1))
 (via (at 97 94) (size 0.6) (drill 0.3) (layers F.Cu B.Cu) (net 1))
 (segment (start 96.1 94) (end 97 94) (width 0.25) (layer B.Cu) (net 1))
 (segment (start 94 95.13) (end 94.97 95.13) (width 0.25) (layer B.Cu) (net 1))
 (via (at 95.1 95.2) (size 0.6) (drill 0.3) (layers F.Cu B.Cu) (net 1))
 (segment (start 94.84 95.46) (end 95.1 95.2) (width 0.25) (layer F.Cu) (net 1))
 (segment (start 94.54 95.46) (end 94.84 95.46) (width 0.25) (layer F.Cu) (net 1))
 (segment (start 95.1 95.2) (end 96.1 94) (width 0.25) (layer B.Cu) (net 1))
 (segment (start 94.97 95.13) (end 95.1 95.2) (width 0.25) (layer B.Cu) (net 1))
 (segment (start 95.81 84.638) (end 95.81 83.51) (width 0.25) (layer F.Cu) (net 6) (status 400000))
 (segment (start 95.556 83.256) (end 95.556 82.483) (width 0.25) (layer F.Cu) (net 6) (status 800000))
 (segment (start 95.81 83.51) (end 95.556 83.256) (width 0.25) (layer F.Cu) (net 6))
 (segment (start 95.81 84.638) (end 95.81 86.9) (width 0.25) (layer F.Cu) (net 6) (status 400000))
 (segment (start 95.81 86.9) (end 95.81 86.91) (width 0.25) (layer F.Cu) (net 6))
 (segment (start 96.09 87.19) (end 98.35 87.19) (width 0.25) (layer F.Cu) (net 6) (status 800000))
 (segment (start 95.81 86.91) (end 96.09 87.19) (width 0.25) (layer F.Cu) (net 6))
 (segment (start 85.65 87.19) (end 95.53 87.19) (width 0.25) (layer F.Cu) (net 6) (status 400000))
 (segment (start 95.53 87.19) (end 95.81 86.91) (width 0.25) (layer F.Cu) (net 6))
 (segment (start 99.15 87.19) (end 98.35 87.19) (width 0.25) (layer B.Cu) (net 6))
 (segment (start 99.7 87.74) (end 99.15 87.19) (width 0.25) (layer B.Cu) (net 6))
 (segment (start 99.7 91.7) (end 99.7 87.74) (width 0.25) (layer B.Cu) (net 6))
 (segment (start 99.8 91.8) (end 99.7 91.7) (width 0.25) (layer B.Cu) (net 6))
 (segment (start 99.8 97.842478) (end 99.8 91.8) (width 0.25) (layer B.Cu) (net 6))
 (segment (start 91.1 100.6) (end 91.25 100.65) (width 0.25) (layer F.Cu) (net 6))
 (segment (start 98.942478 98.7) (end 99.8 97.842478) (width 0.25) (layer B.Cu) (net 6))
 (segment (start 96.9 98.7) (end 98.942478 98.7) (width 0.25) (layer B.Cu) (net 6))
 (segment (start 94.500001 101.099999) (end 96.9 98.7) (width 0.25) (layer B.Cu) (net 6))
 (segment (start 91.1 100.6) (end 91.699999 101.099999) (width 0.25) (layer B.Cu) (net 6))
 (segment (start 91.699999 101.099999) (end 94.500001 101.099999) (width 0.25) (layer B.Cu) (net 6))
 (segment (start 91.25 100.65) (end 91.25 100.55) (width 0.25) (layer F.Cu) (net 6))
 (segment (start 91.25 100.55) (end 91.25 98.264) (width 0.25) (layer F.Cu) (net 6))
 (via (at 91.1 100.6) (size 0.6) (drill 0.3) (layers F.Cu B.Cu) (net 6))
 (segment (start 94.54 84.638) (end 94.54 83.54) (width 0.25) (layer F.Cu) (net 7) (status 400000))
 (segment (start 94.032 83.032) (end 94.032 82.483) (width 0.25) (layer F.Cu) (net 7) (status 800000))
 (segment (start 94.54 83.54) (end 94.032 83.032) (width 0.25) (layer F.Cu) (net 7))
 (segment (start 94.032 82.483) (end 94.032 81.868) (width 0.25) (layer F.Cu) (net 7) (status 400000))
 (segment (start 96.95 84.65) (end 98.35 84.65) (width 0.25) (layer F.Cu) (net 7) (status 800000))
 (segment (start 96.9 84.6) (end 96.95 84.65) (width 0.25) (layer F.Cu) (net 7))
 (segment (start 96.9 81.9) (end 96.9 84.6) (width 0.25) (layer F.Cu) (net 7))
 (segment (start 96.6 81.6) (end 96.9 81.9) (width 0.25) (layer F.Cu) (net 7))
 (segment (start 94.3 81.6) (end 96.6 81.6) (width 0.25) (layer F.Cu) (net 7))
 (segment (start 94.032 81.868) (end 94.3 81.6) (width 0.25) (layer F.Cu) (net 7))
 (segment (start 94.032 82.483) (end 87.617 82.483) (width 0.25) (layer F.Cu) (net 7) (status 400000))
 (segment (start 86.85 84.65) (end 85.65 84.65) (width 0.25) (layer F.Cu) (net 7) (status 800000))
 (segment (start 87 84.5) (end 86.85 84.65) (width 0.25) (layer F.Cu) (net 7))
 (segment (start 87 83.1) (end 87 84.5) (width 0.25) (layer F.Cu) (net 7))
 (segment (start 87.617 82.483) (end 87 83.1) (width 0.25) (layer F.Cu) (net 7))
 (segment (start 90.75 98.264) (end 90.75 99.65) (width 0.25) (layer F.Cu) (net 7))
 (via (at 90.4 100) (size 0.6) (drill 0.3) (layers F.Cu B.Cu) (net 7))
 (segment (start 90.75 99.65) (end 90.4 100) (width 0.25) (layer F.Cu) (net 7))
 (segment (start 90.4 100) (end 87.1 96.7) (width 0.25) (layer B.Cu) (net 7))
 (segment (start 87.1 96.7) (end 86.5 96.1) (width 0.25) (layer B.Cu) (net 7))
 (via (at 84.2 94) (size 0.6) (drill 0.3) (layers F.Cu B.Cu) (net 7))
 (segment (start 84.2 95.302478) (end 84.2 94) (width 0.25) (layer B.Cu) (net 7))
 (segment (start 84.997522 96.1) (end 84.2 95.302478) (width 0.25) (layer B.Cu) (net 7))
 (segment (start 86.5 96.1) (end 84.997522 96.1) (width 0.25) (layer B.Cu) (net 7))
 (segment (start 84.85 84.65) (end 85.65 84.65) (width 0.25) (layer F.Cu) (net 7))
 (segment (start 84.2 85.3) (end 84.85 84.65) (width 0.25) (layer F.Cu) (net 7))
 (segment (start 84.2 94) (end 84.2 85.3) (width 0.25) (layer F.Cu) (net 7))
 (segment (start 92 95.13) (end 92 96.2) (width 0.25) (layer B.Cu) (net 3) (status 400000))
 (segment (start 97.09 94.81) (end 98.35 94.81) (width 0.25) (layer B.Cu) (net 3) (status 800000))
 (segment (start 95.4 96.5) (end 97.09 94.81) (width 0.25) (layer B.Cu) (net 3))
 (segment (start 92.3 96.5) (end 92.8 96.5) (width 0.25) (layer B.Cu) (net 3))
 (segment (start 92.8 96.5) (end 95.4 96.5) (width 0.25) (layer B.Cu) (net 3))
 (segment (start 92 96.2) (end 92.3 96.5) (width 0.25) (layer B.Cu) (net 3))
 (segment (start 85.65 94.81) (end 86.91 94.81) (width 0.25) (layer B.Cu) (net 3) (status 400000))
 (segment (start 91.8 96.4) (end 92 96.2) (width 0.25) (layer B.Cu) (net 3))
 (segment (start 88.5 96.4) (end 91.8 96.4) (width 0.25) (layer B.Cu) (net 3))
 (segment (start 86.91 94.81) (end 88.5 96.4) (width 0.25) (layer B.Cu) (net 3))
 (segment (start 92.75 98.264) (end 92.75 96.55) (width 0.25) (layer F.Cu) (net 3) (status 400000))
 (via (at 92.8 96.5) (size 0.6) (drill 0.3) (layers F.Cu B.Cu) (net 3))
 (segment (start 92.75 96.55) (end 92.8 96.5) (width 0.25) (layer F.Cu) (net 3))
 (segment (start 98.35 92.27) (end 96.53 92.27) (width 0.25) (layer B.Cu) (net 4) (status 400000))
 (segment (start 92 92.7) (end 92 91.32) (width 0.25) (layer B.Cu) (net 4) (status 800000))
 (segment (start 92.5 93.2) (end 92 92.7) (width 0.25) (layer B.Cu) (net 4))
 (segment (start 95.6 93.2) (end 92.5 93.2) (width 0.25) (layer B.Cu) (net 4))
 (segment (start 96.53 92.27) (end 95.6 93.2) (width 0.25) (layer B.Cu) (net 4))
 (segment (start 85.65 92.27) (end 86.67 92.27) (width 0.25) (layer B.Cu) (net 4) (status 400000))
 (segment (start 91.4 93.3) (end 92 92.7) (width 0.25) (layer B.Cu) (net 4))
 (segment (start 87.7 93.3) (end 91.4 93.3) (width 0.25) (layer B.Cu) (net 4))
 (segment (start 92.25 98.264) (end 92.25 99.45) (width 0.25) (layer F.Cu) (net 4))
 (via (at 92.25 99.45) (size 0.6) (drill 0.3) (layers F.Cu B.Cu) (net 4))
 (segment (start 91.825736 99.45) (end 90.475736 98.1) (width 0.25) (layer B.Cu) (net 4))
 (segment (start 92.25 99.45) (end 91.825736 99.45) (width 0.25) (layer B.Cu) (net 4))
 (segment (start 90.475736 98.1) (end 89.7 98.1) (width 0.25) (layer B.Cu) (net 4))
 (via (at 88.7 97.1) (size 0.6) (drill 0.3) (layers F.Cu B.Cu) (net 4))
 (segment (start 89.7 98.1) (end 88.7 97.1) (width 0.25) (layer B.Cu) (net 4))
 (segment (start 88.81501 95.009758) (end 88.81501 92.31501) (width 0.25) (layer F.Cu) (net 4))
 (segment (start 88.7 95.124768) (end 88.81501 95.009758) (width 0.25) (layer F.Cu) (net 4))
 (segment (start 88.7 97.1) (end 88.7 95.124768) (width 0.25) (layer F.Cu) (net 4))
 (via (at 87.9 92.1) (size 0.6) (drill 0.3) (layers F.Cu B.Cu) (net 4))
 (segment (start 88.6 92.1) (end 87.9 92.1) (width 0.25) (layer F.Cu) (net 4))
 (segment (start 88.81501 92.31501) (end 88.6 92.1) (width 0.25) (layer F.Cu) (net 4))
 (segment (start 87.9 92.1) (end 87.2 92.8) (width 0.25) (layer B.Cu) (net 4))
 (segment (start 87.2 92.8) (end 87.7 93.3) (width 0.25) (layer B.Cu) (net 4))
 (segment (start 86.67 92.27) (end 87.2 92.8) (width 0.25) (layer B.Cu) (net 4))
 (segment (start 92 87.51) (end 92 88.9) (width 0.25) (layer B.Cu) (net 5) (status 400000))
 (segment (start 96.73 89.73) (end 98.35 89.73) (width 0.25) (layer B.Cu) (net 5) (status 800000))
 (segment (start 96.5 89.5) (end 96.73 89.73) (width 0.25) (layer B.Cu) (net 5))
 (segment (start 92.6 89.5) (end 96.5 89.5) (width 0.25) (layer B.Cu) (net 5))
 (segment (start 92 88.9) (end 92.6 89.5) (width 0.25) (layer B.Cu) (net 5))
 (segment (start 85.65 89.73) (end 87.87 89.73) (width 0.25) (layer B.Cu) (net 5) (status 400000))
 (segment (start 91.4 89.5) (end 92 88.9) (width 0.25) (layer B.Cu) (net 5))
 (segment (start 87.87 89.73) (end 88.1 89.5) (width 0.25) (layer B.Cu) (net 5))
 (segment (start 91.72501 98.22501) (end 91.72501 96.42501) (width 0.25) (layer F.Cu) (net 5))
 (segment (start 91.75 98.25) (end 91.72501 98.22501) (width 0.25) (layer F.Cu) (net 5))
 (segment (start 91.75 98.264) (end 91.75 98.25) (width 0.25) (layer F.Cu) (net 5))
 (segment (start 91.37499 96.07499) (end 91.37499 90.47499) (width 0.25) (layer F.Cu) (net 5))
 (segment (start 91.72501 96.42501) (end 91.37499 96.07499) (width 0.25) (layer F.Cu) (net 5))
 (segment (start 91.37499 90.47499) (end 90.7 89.8) (width 0.25) (layer F.Cu) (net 5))
 (segment (start 90.7 89.5) (end 91.4 89.5) (width 0.25) (layer B.Cu) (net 5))
 (via (at 90.7 89.5) (size 0.6) (drill 0.3) (layers F.Cu B.Cu) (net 5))
 (segment (start 90.7 89.8) (end 90.7 89.5) (width 0.25) (layer F.Cu) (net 5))
 (segment (start 88.1 89.5) (end 90.7 89.5) (width 0.25) (layer B.Cu) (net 5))
 (segment (start 94.2 100.3) (end 92.2 100.3) (width 0.25) (layer B.Cu) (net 10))
 (via (at 92.2 100.3) (size 0.6) (drill 0.3) (layers F.Cu B.Cu) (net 10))
 (segment (start 92.325002 100.3) (end 92.925002 99.7) (width 0.25) (layer F.Cu) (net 10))
 (segment (start 92.2 100.3) (end 92.325002 100.3) (width 0.25) (layer F.Cu) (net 10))
 (segment (start 93.27499 98.28899) (end 93.25 98.264) (width 0.25) (layer F.Cu) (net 10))
 (segment (start 93.27499 98.92501) (end 93.27499 98.28899) (width 0.25) (layer F.Cu) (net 10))
 (segment (start 92.925002 99.274998) (end 93.27499 98.92501) (width 0.25) (layer F.Cu) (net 10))
 (segment (start 92.925002 99.7) (end 92.925002 99.274998) (width 0.25) (layer F.Cu) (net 10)))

